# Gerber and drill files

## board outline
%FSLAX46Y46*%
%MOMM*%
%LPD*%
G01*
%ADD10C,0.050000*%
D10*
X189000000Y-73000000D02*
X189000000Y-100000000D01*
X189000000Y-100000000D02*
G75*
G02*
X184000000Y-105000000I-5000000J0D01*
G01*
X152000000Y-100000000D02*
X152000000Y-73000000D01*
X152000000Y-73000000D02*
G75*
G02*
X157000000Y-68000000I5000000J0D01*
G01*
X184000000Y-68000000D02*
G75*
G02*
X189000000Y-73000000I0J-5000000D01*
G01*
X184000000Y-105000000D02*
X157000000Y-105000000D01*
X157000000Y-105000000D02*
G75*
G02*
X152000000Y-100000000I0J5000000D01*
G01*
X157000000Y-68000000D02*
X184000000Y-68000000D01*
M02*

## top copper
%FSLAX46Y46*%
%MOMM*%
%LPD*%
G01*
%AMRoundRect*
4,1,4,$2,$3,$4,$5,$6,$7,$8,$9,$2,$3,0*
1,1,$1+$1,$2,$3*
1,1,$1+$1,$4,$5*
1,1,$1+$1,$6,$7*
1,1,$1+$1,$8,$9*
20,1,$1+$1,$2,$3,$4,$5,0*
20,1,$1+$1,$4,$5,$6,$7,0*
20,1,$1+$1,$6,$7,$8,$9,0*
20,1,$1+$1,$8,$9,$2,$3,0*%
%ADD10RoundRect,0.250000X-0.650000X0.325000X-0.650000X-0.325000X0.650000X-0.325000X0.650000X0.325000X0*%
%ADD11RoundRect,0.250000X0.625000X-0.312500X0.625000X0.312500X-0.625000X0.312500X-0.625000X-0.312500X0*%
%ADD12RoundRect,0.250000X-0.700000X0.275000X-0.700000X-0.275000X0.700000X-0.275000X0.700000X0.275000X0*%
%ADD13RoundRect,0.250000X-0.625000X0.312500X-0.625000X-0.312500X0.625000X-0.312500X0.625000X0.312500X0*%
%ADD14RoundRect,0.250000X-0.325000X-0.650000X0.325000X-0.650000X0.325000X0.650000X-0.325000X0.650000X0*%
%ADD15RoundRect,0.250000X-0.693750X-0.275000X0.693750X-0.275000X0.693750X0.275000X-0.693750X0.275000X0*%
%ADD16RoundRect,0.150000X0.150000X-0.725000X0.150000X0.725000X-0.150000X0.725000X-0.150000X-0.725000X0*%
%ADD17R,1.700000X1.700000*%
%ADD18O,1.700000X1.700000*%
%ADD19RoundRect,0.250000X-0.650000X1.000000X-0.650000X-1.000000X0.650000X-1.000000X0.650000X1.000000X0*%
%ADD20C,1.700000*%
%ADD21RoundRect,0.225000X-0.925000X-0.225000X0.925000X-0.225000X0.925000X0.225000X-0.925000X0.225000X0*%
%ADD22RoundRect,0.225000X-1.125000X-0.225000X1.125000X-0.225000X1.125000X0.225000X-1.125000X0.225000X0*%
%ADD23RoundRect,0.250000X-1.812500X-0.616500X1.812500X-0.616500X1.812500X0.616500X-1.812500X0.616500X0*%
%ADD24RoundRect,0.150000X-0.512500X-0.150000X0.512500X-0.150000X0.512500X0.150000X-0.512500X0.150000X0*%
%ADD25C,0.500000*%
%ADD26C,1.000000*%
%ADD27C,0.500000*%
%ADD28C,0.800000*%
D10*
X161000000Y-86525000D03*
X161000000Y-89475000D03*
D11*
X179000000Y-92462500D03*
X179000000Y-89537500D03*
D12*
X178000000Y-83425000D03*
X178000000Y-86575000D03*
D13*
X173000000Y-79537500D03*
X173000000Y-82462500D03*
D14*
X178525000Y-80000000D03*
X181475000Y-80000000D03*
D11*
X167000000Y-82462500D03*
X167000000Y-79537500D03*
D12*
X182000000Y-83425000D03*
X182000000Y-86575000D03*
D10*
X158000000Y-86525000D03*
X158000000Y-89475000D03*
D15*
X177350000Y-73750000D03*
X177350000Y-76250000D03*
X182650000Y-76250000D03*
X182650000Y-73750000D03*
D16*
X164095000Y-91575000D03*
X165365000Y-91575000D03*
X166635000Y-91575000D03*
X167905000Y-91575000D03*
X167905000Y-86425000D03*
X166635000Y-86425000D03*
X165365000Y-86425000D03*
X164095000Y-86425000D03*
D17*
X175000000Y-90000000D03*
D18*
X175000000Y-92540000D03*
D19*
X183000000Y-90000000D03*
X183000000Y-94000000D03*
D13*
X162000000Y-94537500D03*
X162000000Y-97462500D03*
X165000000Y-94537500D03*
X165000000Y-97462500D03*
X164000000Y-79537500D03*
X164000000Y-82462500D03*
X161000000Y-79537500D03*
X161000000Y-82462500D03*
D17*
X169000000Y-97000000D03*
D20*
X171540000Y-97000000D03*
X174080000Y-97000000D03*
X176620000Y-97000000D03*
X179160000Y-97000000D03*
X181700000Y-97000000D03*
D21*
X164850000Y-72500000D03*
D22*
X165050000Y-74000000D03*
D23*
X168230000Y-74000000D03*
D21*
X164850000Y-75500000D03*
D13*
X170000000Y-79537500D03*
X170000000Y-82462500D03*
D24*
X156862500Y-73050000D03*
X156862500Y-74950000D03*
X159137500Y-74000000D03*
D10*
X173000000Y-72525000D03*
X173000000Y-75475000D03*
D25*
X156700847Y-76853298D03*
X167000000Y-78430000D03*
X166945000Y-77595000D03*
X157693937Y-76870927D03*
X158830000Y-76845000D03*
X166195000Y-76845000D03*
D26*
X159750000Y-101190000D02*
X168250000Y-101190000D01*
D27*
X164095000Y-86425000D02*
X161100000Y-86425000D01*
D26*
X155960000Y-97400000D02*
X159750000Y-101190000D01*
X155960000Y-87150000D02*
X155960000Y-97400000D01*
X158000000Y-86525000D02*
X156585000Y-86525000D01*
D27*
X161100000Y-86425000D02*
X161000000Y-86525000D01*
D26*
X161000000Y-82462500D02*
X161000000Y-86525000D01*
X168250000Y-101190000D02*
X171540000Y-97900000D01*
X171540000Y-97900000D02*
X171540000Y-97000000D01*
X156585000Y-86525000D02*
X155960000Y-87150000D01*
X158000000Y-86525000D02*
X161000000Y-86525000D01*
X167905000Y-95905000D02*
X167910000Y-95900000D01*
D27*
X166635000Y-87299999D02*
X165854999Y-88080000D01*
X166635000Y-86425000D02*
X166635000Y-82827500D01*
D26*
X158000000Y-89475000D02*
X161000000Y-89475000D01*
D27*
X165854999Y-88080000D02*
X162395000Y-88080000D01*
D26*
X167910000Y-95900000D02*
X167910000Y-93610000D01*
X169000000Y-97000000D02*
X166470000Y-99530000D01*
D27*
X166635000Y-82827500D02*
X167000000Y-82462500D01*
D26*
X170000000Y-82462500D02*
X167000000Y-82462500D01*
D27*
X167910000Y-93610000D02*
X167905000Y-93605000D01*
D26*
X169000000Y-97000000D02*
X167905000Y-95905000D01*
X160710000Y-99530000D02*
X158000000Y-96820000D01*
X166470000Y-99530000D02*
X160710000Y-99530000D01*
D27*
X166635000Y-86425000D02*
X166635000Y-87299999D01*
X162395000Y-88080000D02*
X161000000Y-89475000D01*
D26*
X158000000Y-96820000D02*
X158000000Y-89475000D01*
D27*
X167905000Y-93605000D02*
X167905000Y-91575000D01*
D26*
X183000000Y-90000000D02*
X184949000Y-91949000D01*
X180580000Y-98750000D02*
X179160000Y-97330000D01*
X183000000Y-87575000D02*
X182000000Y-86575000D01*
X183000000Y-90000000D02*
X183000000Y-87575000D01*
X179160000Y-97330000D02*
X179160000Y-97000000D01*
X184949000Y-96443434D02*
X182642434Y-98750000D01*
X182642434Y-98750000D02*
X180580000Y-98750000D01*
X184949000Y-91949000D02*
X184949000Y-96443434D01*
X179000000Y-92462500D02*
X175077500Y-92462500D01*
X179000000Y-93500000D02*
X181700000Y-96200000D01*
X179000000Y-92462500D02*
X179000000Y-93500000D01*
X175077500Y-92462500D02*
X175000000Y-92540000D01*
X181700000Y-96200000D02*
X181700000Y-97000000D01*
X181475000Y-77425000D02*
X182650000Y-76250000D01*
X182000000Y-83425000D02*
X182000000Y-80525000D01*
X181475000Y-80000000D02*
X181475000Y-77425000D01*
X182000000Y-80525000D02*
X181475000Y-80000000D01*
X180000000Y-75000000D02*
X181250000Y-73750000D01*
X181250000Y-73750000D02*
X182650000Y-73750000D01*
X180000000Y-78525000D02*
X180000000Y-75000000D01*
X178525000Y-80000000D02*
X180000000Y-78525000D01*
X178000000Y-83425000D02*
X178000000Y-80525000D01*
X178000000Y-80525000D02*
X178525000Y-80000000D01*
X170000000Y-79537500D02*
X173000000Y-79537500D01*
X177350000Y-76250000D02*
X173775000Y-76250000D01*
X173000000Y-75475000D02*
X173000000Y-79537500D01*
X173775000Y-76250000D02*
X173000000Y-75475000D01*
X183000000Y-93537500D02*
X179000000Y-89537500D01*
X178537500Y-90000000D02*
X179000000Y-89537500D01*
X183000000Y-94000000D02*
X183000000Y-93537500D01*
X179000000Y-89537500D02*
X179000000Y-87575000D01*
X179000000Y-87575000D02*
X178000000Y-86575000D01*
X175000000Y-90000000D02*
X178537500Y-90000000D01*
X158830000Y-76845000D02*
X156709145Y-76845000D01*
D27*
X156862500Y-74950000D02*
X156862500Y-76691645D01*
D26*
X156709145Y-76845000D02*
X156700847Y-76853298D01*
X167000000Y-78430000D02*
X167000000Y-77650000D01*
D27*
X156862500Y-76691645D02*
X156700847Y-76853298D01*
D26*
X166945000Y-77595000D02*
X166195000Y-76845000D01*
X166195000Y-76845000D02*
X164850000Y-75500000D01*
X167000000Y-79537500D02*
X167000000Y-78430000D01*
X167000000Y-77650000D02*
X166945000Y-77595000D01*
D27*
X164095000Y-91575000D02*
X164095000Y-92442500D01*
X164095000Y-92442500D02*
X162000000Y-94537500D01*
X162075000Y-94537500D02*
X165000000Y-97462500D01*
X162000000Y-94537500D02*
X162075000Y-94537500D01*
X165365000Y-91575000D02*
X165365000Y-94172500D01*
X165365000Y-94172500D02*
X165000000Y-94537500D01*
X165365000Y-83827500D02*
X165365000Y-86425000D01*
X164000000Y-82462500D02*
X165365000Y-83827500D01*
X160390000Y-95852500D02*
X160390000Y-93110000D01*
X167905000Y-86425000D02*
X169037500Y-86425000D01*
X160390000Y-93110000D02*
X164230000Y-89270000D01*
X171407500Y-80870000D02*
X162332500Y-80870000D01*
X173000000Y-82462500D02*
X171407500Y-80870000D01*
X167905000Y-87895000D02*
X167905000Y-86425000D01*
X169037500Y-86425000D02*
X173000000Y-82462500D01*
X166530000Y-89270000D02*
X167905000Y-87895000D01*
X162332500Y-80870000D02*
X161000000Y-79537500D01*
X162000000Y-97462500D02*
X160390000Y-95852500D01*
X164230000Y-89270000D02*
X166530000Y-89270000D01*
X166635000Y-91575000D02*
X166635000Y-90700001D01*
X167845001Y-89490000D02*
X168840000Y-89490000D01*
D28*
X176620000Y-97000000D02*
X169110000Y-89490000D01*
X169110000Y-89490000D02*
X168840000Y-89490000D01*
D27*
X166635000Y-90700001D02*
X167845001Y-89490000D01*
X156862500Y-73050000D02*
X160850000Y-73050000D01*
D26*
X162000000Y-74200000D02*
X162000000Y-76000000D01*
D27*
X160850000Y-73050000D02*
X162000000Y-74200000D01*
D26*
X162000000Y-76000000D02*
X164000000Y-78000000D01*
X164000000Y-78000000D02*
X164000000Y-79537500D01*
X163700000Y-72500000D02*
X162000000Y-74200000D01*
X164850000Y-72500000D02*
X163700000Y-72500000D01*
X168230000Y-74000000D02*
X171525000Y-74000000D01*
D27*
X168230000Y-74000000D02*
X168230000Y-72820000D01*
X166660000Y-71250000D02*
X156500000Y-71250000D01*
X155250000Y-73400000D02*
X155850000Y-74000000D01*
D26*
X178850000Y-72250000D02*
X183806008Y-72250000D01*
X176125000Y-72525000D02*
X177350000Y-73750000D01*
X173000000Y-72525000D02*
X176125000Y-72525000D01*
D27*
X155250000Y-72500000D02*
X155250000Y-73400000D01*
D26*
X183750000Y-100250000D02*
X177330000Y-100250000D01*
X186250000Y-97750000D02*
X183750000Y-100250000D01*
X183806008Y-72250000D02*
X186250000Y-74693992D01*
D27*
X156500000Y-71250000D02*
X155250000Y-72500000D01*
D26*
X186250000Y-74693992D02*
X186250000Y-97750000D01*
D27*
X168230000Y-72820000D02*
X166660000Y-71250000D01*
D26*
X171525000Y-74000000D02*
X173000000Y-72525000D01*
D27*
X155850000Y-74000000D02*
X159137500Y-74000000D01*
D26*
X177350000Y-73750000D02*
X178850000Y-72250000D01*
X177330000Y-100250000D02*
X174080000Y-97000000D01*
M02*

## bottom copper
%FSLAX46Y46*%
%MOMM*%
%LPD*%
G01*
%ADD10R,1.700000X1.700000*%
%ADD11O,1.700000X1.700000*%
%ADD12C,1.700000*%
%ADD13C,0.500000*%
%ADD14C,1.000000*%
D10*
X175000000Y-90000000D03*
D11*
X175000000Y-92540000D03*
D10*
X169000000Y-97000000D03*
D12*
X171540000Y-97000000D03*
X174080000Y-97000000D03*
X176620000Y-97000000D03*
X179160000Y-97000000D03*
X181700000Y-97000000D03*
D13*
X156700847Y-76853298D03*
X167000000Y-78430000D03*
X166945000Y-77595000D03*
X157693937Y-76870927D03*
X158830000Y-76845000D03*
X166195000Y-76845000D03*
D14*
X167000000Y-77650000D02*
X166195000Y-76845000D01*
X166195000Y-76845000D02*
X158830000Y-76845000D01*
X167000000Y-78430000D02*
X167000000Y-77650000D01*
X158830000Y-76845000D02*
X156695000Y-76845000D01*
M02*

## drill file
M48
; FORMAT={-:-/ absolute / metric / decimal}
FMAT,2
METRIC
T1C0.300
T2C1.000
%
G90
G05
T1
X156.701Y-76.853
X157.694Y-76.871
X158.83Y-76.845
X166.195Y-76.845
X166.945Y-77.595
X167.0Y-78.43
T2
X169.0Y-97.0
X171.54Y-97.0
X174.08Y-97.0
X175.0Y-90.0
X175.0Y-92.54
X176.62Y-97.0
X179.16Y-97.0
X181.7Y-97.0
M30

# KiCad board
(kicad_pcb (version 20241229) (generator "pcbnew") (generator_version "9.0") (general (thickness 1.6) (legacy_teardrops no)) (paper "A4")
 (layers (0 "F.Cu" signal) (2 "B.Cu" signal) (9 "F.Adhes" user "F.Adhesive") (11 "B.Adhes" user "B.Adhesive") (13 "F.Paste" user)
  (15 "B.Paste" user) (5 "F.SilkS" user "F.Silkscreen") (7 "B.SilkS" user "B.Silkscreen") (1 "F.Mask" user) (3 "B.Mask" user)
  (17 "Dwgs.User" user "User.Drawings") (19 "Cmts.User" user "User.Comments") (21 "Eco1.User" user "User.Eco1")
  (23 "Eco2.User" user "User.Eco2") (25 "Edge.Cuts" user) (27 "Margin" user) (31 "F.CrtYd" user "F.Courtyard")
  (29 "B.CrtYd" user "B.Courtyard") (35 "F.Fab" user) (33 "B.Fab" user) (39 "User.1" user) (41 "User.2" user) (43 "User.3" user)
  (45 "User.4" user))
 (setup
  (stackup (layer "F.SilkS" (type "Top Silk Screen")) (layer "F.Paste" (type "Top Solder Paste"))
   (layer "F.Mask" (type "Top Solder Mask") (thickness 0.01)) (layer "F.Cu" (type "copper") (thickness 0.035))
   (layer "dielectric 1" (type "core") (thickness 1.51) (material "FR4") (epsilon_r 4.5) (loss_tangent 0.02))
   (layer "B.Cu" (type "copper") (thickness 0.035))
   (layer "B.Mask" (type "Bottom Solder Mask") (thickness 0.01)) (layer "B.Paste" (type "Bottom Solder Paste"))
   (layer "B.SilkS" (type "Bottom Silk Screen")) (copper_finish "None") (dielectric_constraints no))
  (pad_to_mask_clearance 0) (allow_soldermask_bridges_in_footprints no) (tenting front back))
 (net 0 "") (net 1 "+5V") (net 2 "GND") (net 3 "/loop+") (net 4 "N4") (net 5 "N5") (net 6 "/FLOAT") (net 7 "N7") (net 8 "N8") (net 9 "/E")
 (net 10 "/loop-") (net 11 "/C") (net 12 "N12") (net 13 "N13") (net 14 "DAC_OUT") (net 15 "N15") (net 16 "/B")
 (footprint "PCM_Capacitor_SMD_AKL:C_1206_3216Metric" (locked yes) (layer "F.Cu") (at 161 88 -90)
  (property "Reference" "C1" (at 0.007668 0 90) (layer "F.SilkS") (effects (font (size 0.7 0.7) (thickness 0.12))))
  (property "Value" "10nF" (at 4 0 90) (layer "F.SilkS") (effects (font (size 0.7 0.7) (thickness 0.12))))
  (pad "1" smd roundrect (at -1.475 0 270) (size 1.15 1.8) (layers "F.Cu" "F.Mask" "F.Paste") (roundrect_rratio 0.217391) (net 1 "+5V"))
  (pad "2" smd roundrect (at 1.475 0 270) (size 1.15 1.8) (layers "F.Cu" "F.Mask" "F.Paste") (roundrect_rratio 0.217391) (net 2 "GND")))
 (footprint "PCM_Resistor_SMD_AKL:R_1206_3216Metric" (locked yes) (layer "F.Cu") (at 179 91 90)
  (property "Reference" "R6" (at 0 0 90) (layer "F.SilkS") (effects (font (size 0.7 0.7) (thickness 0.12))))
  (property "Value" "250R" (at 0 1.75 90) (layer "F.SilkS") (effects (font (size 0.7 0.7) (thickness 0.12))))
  (pad "1" smd roundrect (at -1.4625 0 90) (size 1.125 1.75) (layers "F.Cu" "F.Mask" "F.Paste") (roundrect_rratio 0.222222) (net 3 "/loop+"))
  (pad "2" smd roundrect (at 1.4625 0 90) (size 1.125 1.75) (layers "F.Cu" "F.Mask" "F.Paste") (roundrect_rratio 0.222222) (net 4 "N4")))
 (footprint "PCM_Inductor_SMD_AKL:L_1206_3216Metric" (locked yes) (layer "F.Cu") (at 178 85 -90)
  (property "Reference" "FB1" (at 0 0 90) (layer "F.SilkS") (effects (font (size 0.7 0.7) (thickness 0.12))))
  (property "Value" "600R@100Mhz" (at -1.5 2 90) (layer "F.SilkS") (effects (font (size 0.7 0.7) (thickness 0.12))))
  (pad "1" smd roundrect (at -1.575 0 270) (size 1.05 1.9) (layers "F.Cu" "F.Mask" "F.Paste") (roundrect_rratio 0.238095) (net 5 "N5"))
  (pad "2" smd roundrect (at 1.575 0 270) (size 1.05 1.9) (layers "F.Cu" "F.Mask" "F.Paste") (roundrect_rratio 0.238095) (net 4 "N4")))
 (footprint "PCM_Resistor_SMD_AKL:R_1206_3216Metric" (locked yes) (layer "F.Cu") (at 173 81 -90)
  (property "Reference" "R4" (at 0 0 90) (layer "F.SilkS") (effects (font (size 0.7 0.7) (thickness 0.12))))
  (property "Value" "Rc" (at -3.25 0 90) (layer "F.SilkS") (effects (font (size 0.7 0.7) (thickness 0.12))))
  (pad "1" smd roundrect (at -1.4625 0 270) (size 1.125 1.75) (layers "F.Cu" "F.Mask" "F.Paste") (roundrect_rratio 0.222222)
   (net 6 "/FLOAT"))
  (pad "2" smd roundrect (at 1.4625 0 270) (size 1.125 1.75) (layers "F.Cu" "F.Mask" "F.Paste") (roundrect_rratio 0.222222) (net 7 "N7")))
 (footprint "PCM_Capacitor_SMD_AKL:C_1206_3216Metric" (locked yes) (layer "F.Cu") (at 180 80)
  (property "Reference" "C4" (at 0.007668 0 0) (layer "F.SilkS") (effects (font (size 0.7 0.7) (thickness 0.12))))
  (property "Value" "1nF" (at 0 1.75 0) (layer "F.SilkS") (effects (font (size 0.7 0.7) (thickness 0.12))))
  (pad "1" smd roundrect (at -1.475 0) (size 1.15 1.8) (layers "F.Cu" "F.Mask" "F.Paste") (roundrect_rratio 0.217391) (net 5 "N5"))
  (pad "2" smd roundrect (at 1.475 0) (size 1.15 1.8) (layers "F.Cu" "F.Mask" "F.Paste") (roundrect_rratio 0.217391) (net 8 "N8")))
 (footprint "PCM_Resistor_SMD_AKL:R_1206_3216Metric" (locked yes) (layer "F.Cu") (at 167 81 90)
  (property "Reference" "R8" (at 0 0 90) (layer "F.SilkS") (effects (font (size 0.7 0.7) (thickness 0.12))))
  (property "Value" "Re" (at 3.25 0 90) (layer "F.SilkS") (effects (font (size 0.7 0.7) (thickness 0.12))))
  (pad "1" smd roundrect (at -1.4625 0 90) (size 1.125 1.75) (layers "F.Cu" "F.Mask" "F.Paste") (roundrect_rratio 0.222222) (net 2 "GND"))
  (pad "2" smd roundrect (at 1.4625 0 90) (size 1.125 1.75) (layers "F.Cu" "F.Mask" "F.Paste") (roundrect_rratio 0.222222) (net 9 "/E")))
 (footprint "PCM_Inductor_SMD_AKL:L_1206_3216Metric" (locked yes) (layer "F.Cu") (at 182 85 -90)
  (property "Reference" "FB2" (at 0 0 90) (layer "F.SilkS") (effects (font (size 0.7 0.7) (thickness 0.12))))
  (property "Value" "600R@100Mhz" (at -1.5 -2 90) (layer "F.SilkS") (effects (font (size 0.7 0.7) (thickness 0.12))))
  (pad "1" smd roundrect (at -1.575 0 270) (size 1.05 1.9) (layers "F.Cu" "F.Mask" "F.Paste") (roundrect_rratio 0.238095) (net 8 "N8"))
  (pad "2" smd roundrect (at 1.575 0 270) (size 1.05 1.9) (layers "F.Cu" "F.Mask" "F.Paste") (roundrect_rratio 0.238095) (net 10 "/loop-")))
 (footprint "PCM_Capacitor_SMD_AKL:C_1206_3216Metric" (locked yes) (layer "F.Cu") (at 158 88 -90)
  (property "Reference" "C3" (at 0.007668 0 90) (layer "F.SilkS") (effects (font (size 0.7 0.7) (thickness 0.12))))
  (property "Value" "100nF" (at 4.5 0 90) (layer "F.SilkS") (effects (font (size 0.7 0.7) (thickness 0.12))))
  (pad "1" smd roundrect (at -1.475 0 270) (size 1.15 1.8) (layers "F.Cu" "F.Mask" "F.Paste") (roundrect_rratio 0.217391) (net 1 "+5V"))
  (pad "2" smd roundrect (at 1.475 0 270) (size 1.15 1.8) (layers "F.Cu" "F.Mask" "F.Paste") (roundrect_rratio 0.217391) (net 2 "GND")))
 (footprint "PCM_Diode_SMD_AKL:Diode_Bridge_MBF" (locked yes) (layer "F.Cu") (at 180 75)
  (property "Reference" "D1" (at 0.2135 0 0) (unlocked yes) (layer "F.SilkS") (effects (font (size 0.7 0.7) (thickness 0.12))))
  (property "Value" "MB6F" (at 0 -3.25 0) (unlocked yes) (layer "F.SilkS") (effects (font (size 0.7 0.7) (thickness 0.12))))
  (pad "1" smd roundrect (at -2.65 -1.25) (size 1.8875 1.05) (layers "F.Cu" "F.Mask" "F.Paste") (roundrect_rratio 0.2380952381)
   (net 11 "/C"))
  (pad "2" smd roundrect (at -2.65 1.25) (size 1.8875 1.05) (layers "F.Cu" "F.Mask" "F.Paste") (roundrect_rratio 0.2380952381)
   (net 6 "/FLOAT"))
  (pad "3" smd roundrect (at 2.65 1.25) (size 1.8875 1.05) (layers "F.Cu" "F.Mask" "F.Paste") (roundrect_rratio 0.2380952381) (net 8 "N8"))
  (pad "4" smd roundrect (at 2.65 -1.25) (size 1.8875 1.05) (layers "F.Cu" "F.Mask" "F.Paste") (roundrect_rratio 0.2380952381) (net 5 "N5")))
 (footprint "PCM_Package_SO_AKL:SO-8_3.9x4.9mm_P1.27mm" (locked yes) (layer "F.Cu") (at 166 89 90)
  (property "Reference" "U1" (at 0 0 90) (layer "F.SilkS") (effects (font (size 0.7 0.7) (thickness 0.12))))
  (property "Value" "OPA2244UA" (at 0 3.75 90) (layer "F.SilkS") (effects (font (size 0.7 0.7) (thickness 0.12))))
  (pad "1" smd roundrect (at -2.575 -1.905 90) (size 1.75 0.6) (layers "F.Cu" "F.Mask" "F.Paste") (roundrect_rratio 0.25) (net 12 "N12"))
  (pad "2" smd roundrect (at -2.575 -0.635 90) (size 1.75 0.6) (layers "F.Cu" "F.Mask" "F.Paste") (roundrect_rratio 0.25) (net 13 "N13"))
  (pad "3" smd roundrect (at -2.575 0.635 90) (size 1.75 0.6) (layers "F.Cu" "F.Mask" "F.Paste") (roundrect_rratio 0.25) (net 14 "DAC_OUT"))
  (pad "4" smd roundrect (at -2.575 1.905 90) (size 1.75 0.6) (layers "F.Cu" "F.Mask" "F.Paste") (roundrect_rratio 0.25) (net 2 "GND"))
  (pad "5" smd roundrect (at 2.575 1.905 90) (size 1.75 0.6) (layers "F.Cu" "F.Mask" "F.Paste") (roundrect_rratio 0.25) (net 7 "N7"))
  (pad "6" smd roundrect (at 2.575 0.635 90) (size 1.75 0.6) (layers "F.Cu" "F.Mask" "F.Paste") (roundrect_rratio 0.25) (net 2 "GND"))
  (pad "7" smd roundrect (at 2.575 -0.635 90) (size 1.75 0.6) (layers "F.Cu" "F.Mask" "F.Paste") (roundrect_rratio 0.25) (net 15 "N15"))
  (pad "8" smd roundrect (at 2.575 -1.905 90) (size 1.75 0.6) (layers "F.Cu" "F.Mask" "F.Paste") (roundrect_rratio 0.25) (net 1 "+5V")))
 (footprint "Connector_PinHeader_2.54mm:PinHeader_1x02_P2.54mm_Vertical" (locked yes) (layer "F.Cu") (at 175 90)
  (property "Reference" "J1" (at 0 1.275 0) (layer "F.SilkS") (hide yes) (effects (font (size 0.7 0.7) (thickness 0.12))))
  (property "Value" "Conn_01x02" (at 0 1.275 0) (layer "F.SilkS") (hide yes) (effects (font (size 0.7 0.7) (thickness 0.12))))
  (pad "1" thru_hole rect (at 0 0) (size 1.7 1.7) (drill 1) (layers "*.Cu" "*.Mask") (remove_unused_layers no) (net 4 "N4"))
  (pad "2" thru_hole oval (at 0 2.54) (size 1.7 1.7) (drill 1) (layers "*.Cu" "*.Mask") (remove_unused_layers no) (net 3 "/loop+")))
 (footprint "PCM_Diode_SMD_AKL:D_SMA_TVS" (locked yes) (layer "F.Cu") (at 183 92 -90)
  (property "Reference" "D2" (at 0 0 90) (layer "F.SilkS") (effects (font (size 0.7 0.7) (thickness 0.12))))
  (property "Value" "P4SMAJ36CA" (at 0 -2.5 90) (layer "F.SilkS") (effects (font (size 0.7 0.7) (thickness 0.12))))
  (pad "1" smd roundrect (at -2 0 270) (size 2.5 1.8) (layers "F.Cu" "F.Mask" "F.Paste") (roundrect_rratio 0.1388888889) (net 10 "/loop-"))
  (pad "2" smd roundrect (at 2 0 270) (size 2.5 1.8) (layers "F.Cu" "F.Mask" "F.Paste") (roundrect_rratio 0.1388888889) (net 4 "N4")))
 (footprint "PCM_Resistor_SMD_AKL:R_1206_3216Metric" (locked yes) (layer "F.Cu") (at 162 96 -90)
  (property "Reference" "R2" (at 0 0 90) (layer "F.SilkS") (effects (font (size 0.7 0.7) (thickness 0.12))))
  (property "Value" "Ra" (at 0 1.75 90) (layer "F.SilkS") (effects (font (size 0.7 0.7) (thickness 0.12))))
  (pad "1" smd roundrect (at -1.4625 0 270) (size 1.125 1.75) (layers "F.Cu" "F.Mask" "F.Paste") (roundrect_rratio 0.222222) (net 12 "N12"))
  (pad "2" smd roundrect (at 1.4625 0 270) (size 1.125 1.75) (layers "F.Cu" "F.Mask" "F.Paste") (roundrect_rratio 0.222222) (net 7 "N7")))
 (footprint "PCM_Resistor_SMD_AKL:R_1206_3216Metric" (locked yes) (layer "F.Cu") (at 165 96 -90)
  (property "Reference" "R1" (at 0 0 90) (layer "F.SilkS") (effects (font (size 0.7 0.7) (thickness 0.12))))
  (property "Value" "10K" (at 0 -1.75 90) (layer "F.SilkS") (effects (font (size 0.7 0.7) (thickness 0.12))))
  (pad "1" smd roundrect (at -1.4625 0 270) (size 1.125 1.75) (layers "F.Cu" "F.Mask" "F.Paste") (roundrect_rratio 0.222222) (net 13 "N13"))
  (pad "2" smd roundrect (at 1.4625 0 270) (size 1.125 1.75) (layers "F.Cu" "F.Mask" "F.Paste") (roundrect_rratio 0.222222) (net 12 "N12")))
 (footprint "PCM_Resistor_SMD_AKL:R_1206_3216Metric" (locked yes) (layer "F.Cu") (at 164 81 -90)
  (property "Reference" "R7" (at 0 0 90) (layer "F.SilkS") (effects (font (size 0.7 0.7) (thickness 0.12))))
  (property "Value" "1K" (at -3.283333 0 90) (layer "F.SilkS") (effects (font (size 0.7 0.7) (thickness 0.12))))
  (pad "1" smd roundrect (at -1.4625 0 270) (size 1.125 1.75) (layers "F.Cu" "F.Mask" "F.Paste") (roundrect_rratio 0.222222) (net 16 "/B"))
  (pad "2" smd roundrect (at 1.4625 0 270) (size 1.125 1.75) (layers "F.Cu" "F.Mask" "F.Paste") (roundrect_rratio 0.222222) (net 15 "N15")))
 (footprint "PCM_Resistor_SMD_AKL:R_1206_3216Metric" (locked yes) (layer "F.Cu") (at 161 81 -90)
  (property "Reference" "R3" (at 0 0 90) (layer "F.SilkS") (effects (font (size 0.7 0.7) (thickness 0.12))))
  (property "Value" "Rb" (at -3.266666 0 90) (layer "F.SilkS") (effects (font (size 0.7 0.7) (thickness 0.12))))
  (pad "1" smd roundrect (at -1.4625 0 270) (size 1.125 1.75) (layers "F.Cu" "F.Mask" "F.Paste") (roundrect_rratio 0.222222) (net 7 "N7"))
  (pad "2" smd roundrect (at 1.4625 0 270) (size 1.125 1.75) (layers "F.Cu" "F.Mask" "F.Paste") (roundrect_rratio 0.222222) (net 1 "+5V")))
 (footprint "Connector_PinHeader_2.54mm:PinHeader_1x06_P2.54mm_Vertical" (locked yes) (layer "F.Cu") (at 169 97 90)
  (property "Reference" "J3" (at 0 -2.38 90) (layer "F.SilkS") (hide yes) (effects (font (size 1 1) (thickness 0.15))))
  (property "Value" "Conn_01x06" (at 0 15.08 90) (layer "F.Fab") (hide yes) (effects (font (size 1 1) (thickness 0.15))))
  (pad "1" thru_hole rect (at 0 0 90) (size 1.7 1.7) (drill 1) (layers "*.Cu" "*.Mask") (remove_unused_layers no) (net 2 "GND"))
  (pad "2" thru_hole circle (at 0 2.54 90) (size 1.7 1.7) (drill 1) (layers "*.Cu" "*.Mask") (remove_unused_layers no) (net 1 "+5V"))
  (pad "3" thru_hole circle (at 0 5.08 90) (size 1.7 1.7) (drill 1) (layers "*.Cu" "*.Mask") (remove_unused_layers no) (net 11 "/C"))
  (pad "4" thru_hole circle (at 0 7.62 90) (size 1.7 1.7) (drill 1) (layers "*.Cu" "*.Mask") (remove_unused_layers no) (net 14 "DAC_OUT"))
  (pad "5" thru_hole circle (at 0 10.16 90) (size 1.7 1.7) (drill 1) (layers "*.Cu" "*.Mask") (remove_unused_layers no) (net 10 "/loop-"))
  (pad "6" thru_hole circle (at 0 12.7 90) (size 1.7 1.7) (drill 1) (layers "*.Cu" "*.Mask") (remove_unused_layers no) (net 3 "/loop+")))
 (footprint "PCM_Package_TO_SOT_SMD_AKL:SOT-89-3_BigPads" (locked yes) (layer "F.Cu") (at 167 74)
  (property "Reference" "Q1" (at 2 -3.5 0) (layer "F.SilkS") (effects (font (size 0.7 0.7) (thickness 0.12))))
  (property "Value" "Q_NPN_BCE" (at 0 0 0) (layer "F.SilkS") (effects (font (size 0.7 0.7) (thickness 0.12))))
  (pad "1" smd roundrect (at -2.15 -1.5) (size 2.3 0.9) (layers "F.Cu" "F.Mask" "F.Paste") (roundrect_rratio 0.25) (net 16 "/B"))
  (pad "2" smd roundrect (at -1.95 0) (size 2.7 0.9) (layers "F.Cu" "F.Mask" "F.Paste") (roundrect_rratio 0.25) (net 11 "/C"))
  (pad "2" smd roundrect (at 1.23 0) (size 4.125 1.733) (layers "F.Cu" "F.Mask" "F.Paste") (roundrect_rratio 0.1442585113) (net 11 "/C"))
  (pad "3" smd roundrect (at -2.15 1.5) (size 2.3 0.9) (layers "F.Cu" "F.Mask" "F.Paste") (roundrect_rratio 0.25) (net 9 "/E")))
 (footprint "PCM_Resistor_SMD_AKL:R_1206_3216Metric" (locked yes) (layer "F.Cu") (at 170 81 -90)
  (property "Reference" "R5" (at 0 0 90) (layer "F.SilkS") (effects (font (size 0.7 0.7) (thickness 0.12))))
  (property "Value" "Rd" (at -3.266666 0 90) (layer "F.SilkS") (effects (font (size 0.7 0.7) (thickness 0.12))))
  (pad "1" smd roundrect (at -1.4625 0 270) (size 1.125 1.75) (layers "F.Cu" "F.Mask" "F.Paste") (roundrect_rratio 0.222222)
   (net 6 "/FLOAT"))
  (pad "2" smd roundrect (at 1.4625 0 270) (size 1.125 1.75) (layers "F.Cu" "F.Mask" "F.Paste") (roundrect_rratio 0.222222) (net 2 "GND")))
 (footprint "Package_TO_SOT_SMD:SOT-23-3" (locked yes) (layer "F.Cu") (at 158 74)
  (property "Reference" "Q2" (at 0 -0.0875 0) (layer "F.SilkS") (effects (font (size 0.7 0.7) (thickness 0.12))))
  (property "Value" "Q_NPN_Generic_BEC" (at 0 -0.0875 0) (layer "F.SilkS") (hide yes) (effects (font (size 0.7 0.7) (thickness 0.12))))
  (pad "1" smd roundrect (at -1.1375 -0.95) (size 1.325 0.6) (layers "F.Cu" "F.Mask" "F.Paste") (roundrect_rratio 0.25) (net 16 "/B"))
  (pad "2" smd roundrect (at -1.1375 0.95) (size 1.325 0.6) (layers "F.Cu" "F.Mask" "F.Paste") (roundrect_rratio 0.25) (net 9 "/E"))
  (pad "3" smd roundrect (at 1.1375 0) (size 1.325 0.6) (layers "F.Cu" "F.Mask" "F.Paste") (roundrect_rratio 0.25) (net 11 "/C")))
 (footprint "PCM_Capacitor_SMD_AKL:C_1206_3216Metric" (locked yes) (layer "F.Cu") (at 173 74 -90)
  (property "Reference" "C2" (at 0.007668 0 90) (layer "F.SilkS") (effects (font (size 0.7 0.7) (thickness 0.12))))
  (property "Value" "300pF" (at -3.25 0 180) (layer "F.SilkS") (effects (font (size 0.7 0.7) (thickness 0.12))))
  (pad "1" smd roundrect (at -1.475 0 270) (size 1.15 1.8) (layers "F.Cu" "F.Mask" "F.Paste") (roundrect_rratio 0.217391) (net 11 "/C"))
  (pad "2" smd roundrect (at 1.475 0 270) (size 1.15 1.8) (layers "F.Cu" "F.Mask" "F.Paste") (roundrect_rratio 0.217391) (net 6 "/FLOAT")))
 (gr_line (start 189 73) (end 189 100) (stroke (width 0.05) (type default)) (locked yes) (layer "Edge.Cuts"))
 (gr_arc (start 189 100) (mid 187.535534 103.535534) (end 184 105) (stroke (width 0.05) (type default)) (locked yes) (layer "Edge.Cuts"))
 (gr_line (start 152 100) (end 152 73) (stroke (width 0.05) (type default)) (locked yes) (layer "Edge.Cuts"))
 (gr_arc (start 152 73) (mid 153.464466 69.464466) (end 157 68) (stroke (width 0.05) (type default)) (locked yes) (layer "Edge.Cuts"))
 (gr_arc (start 184 68) (mid 187.535534 69.464466) (end 189 73) (stroke (width 0.05) (type default)) (locked yes) (layer "Edge.Cuts"))
 (gr_line (start 184 105) (end 157 105) (stroke (width 0.05) (type default)) (locked yes) (layer "Edge.Cuts"))
 (gr_arc (start 157 105) (mid 153.464466 103.535534) (end 152 100) (stroke (width 0.05) (type default)) (locked yes) (layer "Edge.Cuts"))
 (gr_line (start 157 68) (end 184 68) (stroke (width 0.05) (type default)) (locked yes) (layer "Edge.Cuts"))
 (segment (start 159.75 101.19) (end 168.25 101.19) (width 1) (locked yes) (layer "F.Cu") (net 1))
 (segment (start 164.095 86.425) (end 161.1 86.425) (width 0.5) (locked yes) (layer "F.Cu") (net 1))
 (segment (start 155.96 97.4) (end 159.75 101.19) (width 1) (locked yes) (layer "F.Cu") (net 1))
 (segment (start 155.96 87.15) (end 155.96 97.4) (width 1) (locked yes) (layer "F.Cu") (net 1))
 (segment (start 158 86.525) (end 156.585 86.525) (width 1) (locked yes) (layer "F.Cu") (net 1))
 (segment (start 161.1 86.425) (end 161 86.525) (width 0.5) (locked yes) (layer "F.Cu") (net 1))
 (segment (start 161 82.4625) (end 161 86.525) (width 1) (locked yes) (layer "F.Cu") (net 1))
 (segment (start 168.25 101.19) (end 171.54 97.9) (width 1) (locked yes) (layer "F.Cu") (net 1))
 (segment (start 171.54 97.9) (end 171.54 97) (width 1) (locked yes) (layer "F.Cu") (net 1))
 (segment (start 156.585 86.525) (end 155.96 87.15) (width 1) (locked yes) (layer "F.Cu") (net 1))
 (segment (start 158 86.525) (end 161 86.525) (width 1) (locked yes) (layer "F.Cu") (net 1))
 (segment (start 167.905 95.905) (end 167.91 95.9) (width 1) (locked yes) (layer "F.Cu") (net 2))
 (segment (start 166.635 87.299999) (end 165.854999 88.08) (width 0.5) (locked yes) (layer "F.Cu") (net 2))
 (segment (start 166.635 86.425) (end 166.635 82.8275) (width 0.5) (locked yes) (layer "F.Cu") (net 2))
 (segment (start 158 89.475) (end 161 89.475) (width 1) (locked yes) (layer "F.Cu") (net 2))
 (segment (start 165.854999 88.08) (end 162.395 88.08) (width 0.5) (locked yes) (layer "F.Cu") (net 2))
 (segment (start 167.91 95.9) (end 167.91 93.61) (width 1) (locked yes) (layer "F.Cu") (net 2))
 (segment (start 169 97) (end 166.47 99.53) (width 1) (locked yes) (layer "F.Cu") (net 2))
 (segment (start 166.635 82.8275) (end 167 82.4625) (width 0.5) (locked yes) (layer "F.Cu") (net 2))
 (segment (start 170 82.4625) (end 167 82.4625) (width 1) (locked yes) (layer "F.Cu") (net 2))
 (segment (start 167.91 93.61) (end 167.905 93.605) (width 0.5) (locked yes) (layer "F.Cu") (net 2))
 (segment (start 169 97) (end 167.905 95.905) (width 1) (locked yes) (layer "F.Cu") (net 2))
 (segment (start 160.71 99.53) (end 158 96.82) (width 1) (locked yes) (layer "F.Cu") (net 2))
 (segment (start 166.47 99.53) (end 160.71 99.53) (width 1) (locked yes) (layer "F.Cu") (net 2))
 (segment (start 166.635 86.425) (end 166.635 87.299999) (width 0.5) (locked yes) (layer "F.Cu") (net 2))
 (segment (start 162.395 88.08) (end 161 89.475) (width 0.5) (locked yes) (layer "F.Cu") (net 2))
 (segment (start 158 96.82) (end 158 89.475) (width 1) (locked yes) (layer "F.Cu") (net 2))
 (segment (start 167.905 93.605) (end 167.905 91.575) (width 0.5) (locked yes) (layer "F.Cu") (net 2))
 (segment (start 183 90) (end 184.949 91.949) (width 1) (locked yes) (layer "F.Cu") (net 10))
 (segment (start 180.58 98.75) (end 179.16 97.33) (width 1) (locked yes) (layer "F.Cu") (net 10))
 (segment (start 183 87.575) (end 182 86.575) (width 1) (locked yes) (layer "F.Cu") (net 10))
 (segment (start 183 90) (end 183 87.575) (width 1) (locked yes) (layer "F.Cu") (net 10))
 (segment (start 179.16 97.33) (end 179.16 97) (width 1) (locked yes) (layer "F.Cu") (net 10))
 (segment (start 184.949 96.443434) (end 182.642434 98.75) (width 1) (locked yes) (layer "F.Cu") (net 10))
 (segment (start 182.642434 98.75) (end 180.58 98.75) (width 1) (locked yes) (layer "F.Cu") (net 10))
 (segment (start 184.949 91.949) (end 184.949 96.443434) (width 1) (locked yes) (layer "F.Cu") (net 10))
 (segment (start 179 92.4625) (end 175.0775 92.4625) (width 1) (locked yes) (layer "F.Cu") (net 3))
 (segment (start 179 93.5) (end 181.7 96.2) (width 1) (locked yes) (layer "F.Cu") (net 3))
 (segment (start 179 92.4625) (end 179 93.5) (width 1) (locked yes) (layer "F.Cu") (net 3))
 (segment (start 175.0775 92.4625) (end 175 92.54) (width 1) (locked yes) (layer "F.Cu") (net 3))
 (segment (start 181.7 96.2) (end 181.7 97) (width 1) (locked yes) (layer "F.Cu") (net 3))
 (segment (start 181.475 77.425) (end 182.65 76.25) (width 1) (locked yes) (layer "F.Cu") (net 8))
 (segment (start 182 83.425) (end 182 80.525) (width 1) (locked yes) (layer "F.Cu") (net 8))
 (segment (start 181.475 80) (end 181.475 77.425) (width 1) (locked yes) (layer "F.Cu") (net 8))
 (segment (start 182 80.525) (end 181.475 80) (width 1) (locked yes) (layer "F.Cu") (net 8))
 (segment (start 180 75) (end 181.25 73.75) (width 1) (locked yes) (layer "F.Cu") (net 5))
 (segment (start 181.25 73.75) (end 182.65 73.75) (width 1) (locked yes) (layer "F.Cu") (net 5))
 (segment (start 180 78.525) (end 180 75) (width 1) (locked yes) (layer "F.Cu") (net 5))
 (segment (start 178.525 80) (end 180 78.525) (width 1) (locked yes) (layer "F.Cu") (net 5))
 (segment (start 178 83.425) (end 178 80.525) (width 1) (locked yes) (layer "F.Cu") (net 5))
 (segment (start 178 80.525) (end 178.525 80) (width 1) (locked yes) (layer "F.Cu") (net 5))
 (segment (start 170 79.5375) (end 173 79.5375) (width 1) (locked yes) (layer "F.Cu") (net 6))
 (segment (start 177.35 76.25) (end 173.775 76.25) (width 1) (locked yes) (layer "F.Cu") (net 6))
 (segment (start 173 75.475) (end 173 79.5375) (width 1) (locked yes) (layer "F.Cu") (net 6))
 (segment (start 173.775 76.25) (end 173 75.475) (width 1) (locked yes) (layer "F.Cu") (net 6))
 (segment (start 183 93.5375) (end 179 89.5375) (width 1) (locked yes) (layer "F.Cu") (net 4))
 (segment (start 178.5375 90) (end 179 89.5375) (width 1) (locked yes) (layer "F.Cu") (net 4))
 (segment (start 183 94) (end 183 93.5375) (width 1) (locked yes) (layer "F.Cu") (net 4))
 (segment (start 179 89.5375) (end 179 87.575) (width 1) (locked yes) (layer "F.Cu") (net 4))
 (segment (start 179 87.575) (end 178 86.575) (width 1) (locked yes) (layer "F.Cu") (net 4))
 (segment (start 175 90) (end 178.5375 90) (width 1) (locked yes) (layer "F.Cu") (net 4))
 (segment (start 158.83 76.845) (end 156.709145 76.845) (width 1) (locked yes) (layer "F.Cu") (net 9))
 (segment (start 156.8625 74.95) (end 156.8625 76.691645) (width 0.5) (locked yes) (layer "F.Cu") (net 9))
 (segment (start 156.709145 76.845) (end 156.700847 76.853298) (width 1) (locked yes) (layer "F.Cu") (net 9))
 (segment (start 167 78.43) (end 167 77.65) (width 1) (locked yes) (layer "F.Cu") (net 9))
 (segment (start 156.8625 76.691645) (end 156.700847 76.853298) (width 0.5) (locked yes) (layer "F.Cu") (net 9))
 (segment (start 166.945 77.595) (end 166.195 76.845) (width 1) (locked yes) (layer "F.Cu") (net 9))
 (segment (start 166.195 76.845) (end 164.85 75.5) (width 1) (locked yes) (layer "F.Cu") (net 9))
 (segment (start 167 79.5375) (end 167 78.43) (width 1) (locked yes) (layer "F.Cu") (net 9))
 (segment (start 167 77.65) (end 166.945 77.595) (width 1) (locked yes) (layer "F.Cu") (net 9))
 (via (at 156.700847 76.853298) (size 0.5) (drill 0.3) (layers "F.Cu" "B.Cu") (locked yes) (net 9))
 (via (at 167 78.43) (size 0.5) (drill 0.3) (layers "F.Cu" "B.Cu") (locked yes) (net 9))
 (via (at 166.945 77.595) (size 0.5) (drill 0.3) (layers "F.Cu" "B.Cu") (locked yes) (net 9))
 (via (at 157.693937 76.870927) (size 0.5) (drill 0.3) (layers "F.Cu" "B.Cu") (locked yes) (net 9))
 (via (at 158.83 76.845) (size 0.5) (drill 0.3) (layers "F.Cu" "B.Cu") (locked yes) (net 9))
 (via (at 166.195 76.845) (size 0.5) (drill 0.3) (layers "F.Cu" "B.Cu") (locked yes) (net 9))
 (segment (start 167 77.65) (end 166.195 76.845) (width 1) (locked yes) (layer "B.Cu") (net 9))
 (segment (start 166.195 76.845) (end 158.83 76.845) (width 1) (locked yes) (layer "B.Cu") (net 9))
 (segment (start 167 78.43) (end 167 77.65) (width 1) (locked yes) (layer "B.Cu") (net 9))
 (segment (start 158.83 76.845) (end 156.695 76.845) (width 1) (locked yes) (layer "B.Cu") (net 9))
 (segment (start 164.095 91.575) (end 164.095 92.4425) (width 0.5) (locked yes) (layer "F.Cu") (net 12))
 (segment (start 164.095 92.4425) (end 162 94.5375) (width 0.5) (locked yes) (layer "F.Cu") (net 12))
 (segment (start 162.075 94.5375) (end 165 97.4625) (width 0.5) (locked yes) (layer "F.Cu") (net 12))
 (segment (start 162 94.5375) (end 162.075 94.5375) (width 0.5) (locked yes) (layer "F.Cu") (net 12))
 (segment (start 165.365 91.575) (end 165.365 94.1725) (width 0.5) (locked yes) (layer "F.Cu") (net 13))
 (segment (start 165.365 94.1725) (end 165 94.5375) (width 0.5) (locked yes) (layer "F.Cu") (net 13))
 (segment (start 165.365 83.8275) (end 165.365 86.425) (width 0.5) (locked yes) (layer "F.Cu") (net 15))
 (segment (start 164 82.4625) (end 165.365 83.8275) (width 0.5) (locked yes) (layer "F.Cu") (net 15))
 (segment (start 160.39 95.8525) (end 160.39 93.11) (width 0.5) (locked yes) (layer "F.Cu") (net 7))
 (segment (start 167.905 86.425) (end 169.0375 86.425) (width 0.5) (locked yes) (layer "F.Cu") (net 7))
 (segment (start 160.39 93.11) (end 164.23 89.27) (width 0.5) (locked yes) (layer "F.Cu") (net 7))
 (segment (start 171.4075 80.87) (end 162.3325 80.87) (width 0.5) (locked yes) (layer "F.Cu") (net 7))
 (segment (start 173 82.4625) (end 171.4075 80.87) (width 0.5) (locked yes) (layer "F.Cu") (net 7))
 (segment (start 167.905 87.895) (end 167.905 86.425) (width 0.5) (locked yes) (layer "F.Cu") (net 7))
 (segment (start 169.0375 86.425) (end 173 82.4625) (width 0.5) (locked yes) (layer "F.Cu") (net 7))
 (segment (start 166.53 89.27) (end 167.905 87.895) (width 0.5) (locked yes) (layer "F.Cu") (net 7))
 (segment (start 162.3325 80.87) (end 161 79.5375) (width 0.5) (locked yes) (layer "F.Cu") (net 7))
 (segment (start 162 97.4625) (end 160.39 95.8525) (width 0.5) (locked yes) (layer "F.Cu") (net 7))
 (segment (start 164.23 89.27) (end 166.53 89.27) (width 0.5) (locked yes) (layer "F.Cu") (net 7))
 (segment (start 166.635 91.575) (end 166.635 90.700001) (width 0.5) (locked yes) (layer "F.Cu") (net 14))
 (segment (start 167.845001 89.49) (end 168.84 89.49) (width 0.5) (locked yes) (layer "F.Cu") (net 14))
 (segment (start 176.62 97) (end 169.11 89.49) (width 0.8) (locked yes) (layer "F.Cu") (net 14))
 (segment (start 169.11 89.49) (end 168.84 89.49) (width 0.8) (locked yes) (layer "F.Cu") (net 14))
 (segment (start 166.635 90.700001) (end 167.845001 89.49) (width 0.5) (locked yes) (layer "F.Cu") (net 14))
 (segment (start 156.8625 73.05) (end 160.85 73.05) (width 0.5) (locked yes) (layer "F.Cu") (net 16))
 (segment (start 162 74.2) (end 162 76) (width 1) (locked yes) (layer "F.Cu") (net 16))
 (segment (start 160.85 73.05) (end 162 74.2) (width 0.5) (locked yes) (layer "F.Cu") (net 16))
 (segment (start 162 76) (end 164 78) (width 1) (locked yes) (layer "F.Cu") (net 16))
 (segment (start 164 78) (end 164 79.5375) (width 1) (locked yes) (layer "F.Cu") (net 16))
 (segment (start 163.7 72.5) (end 162 74.2) (width 1) (locked yes) (layer "F.Cu") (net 16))
 (segment (start 164.85 72.5) (end 163.7 72.5) (width 1) (locked yes) (layer "F.Cu") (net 16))
 (segment (start 168.23 74) (end 171.525 74) (width 1) (locked yes) (layer "F.Cu") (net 11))
 (segment (start 168.23 74) (end 168.23 72.82) (width 0.5) (locked yes) (layer "F.Cu") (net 11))
 (segment (start 166.66 71.25) (end 156.5 71.25) (width 0.5) (locked yes) (layer "F.Cu") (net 11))
 (segment (start 155.25 73.4) (end 155.85 74) (width 0.5) (locked yes) (layer "F.Cu") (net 11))
 (segment (start 178.85 72.25) (end 183.806008 72.25) (width 1) (locked yes) (layer "F.Cu") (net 11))
 (segment (start 176.125 72.525) (end 177.35 73.75) (width 1) (locked yes) (layer "F.Cu") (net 11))
 (segment (start 173 72.525) (end 176.125 72.525) (width 1) (locked yes) (layer "F.Cu") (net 11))
 (segment (start 155.25 72.5) (end 155.25 73.4) (width 0.5) (locked yes) (layer "F.Cu") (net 11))
 (segment (start 183.75 100.25) (end 177.33 100.25) (width 1) (locked yes) (layer "F.Cu") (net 11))
 (segment (start 186.25 97.75) (end 183.75 100.25) (width 1) (locked yes) (layer "F.Cu") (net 11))
 (segment (start 183.806008 72.25) (end 186.25 74.693992) (width 1) (locked yes) (layer "F.Cu") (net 11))
 (segment (start 156.5 71.25) (end 155.25 72.5) (width 0.5) (locked yes) (layer "F.Cu") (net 11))
 (segment (start 186.25 74.693992) (end 186.25 97.75) (width 1) (locked yes) (layer "F.Cu") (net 11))
 (segment (start 168.23 72.82) (end 166.66 71.25) (width 0.5) (locked yes) (layer "F.Cu") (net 11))
 (segment (start 171.525 74) (end 173 72.525) (width 1) (locked yes) (layer "F.Cu") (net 11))
 (segment (start 155.85 74) (end 159.1375 74) (width 0.5) (locked yes) (layer "F.Cu") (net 11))
 (segment (start 177.35 73.75) (end 178.85 72.25) (width 1) (locked yes) (layer "F.Cu") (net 11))
 (segment (start 177.33 100.25) (end 174.08 97) (width 1) (locked yes) (layer "F.Cu") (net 11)))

